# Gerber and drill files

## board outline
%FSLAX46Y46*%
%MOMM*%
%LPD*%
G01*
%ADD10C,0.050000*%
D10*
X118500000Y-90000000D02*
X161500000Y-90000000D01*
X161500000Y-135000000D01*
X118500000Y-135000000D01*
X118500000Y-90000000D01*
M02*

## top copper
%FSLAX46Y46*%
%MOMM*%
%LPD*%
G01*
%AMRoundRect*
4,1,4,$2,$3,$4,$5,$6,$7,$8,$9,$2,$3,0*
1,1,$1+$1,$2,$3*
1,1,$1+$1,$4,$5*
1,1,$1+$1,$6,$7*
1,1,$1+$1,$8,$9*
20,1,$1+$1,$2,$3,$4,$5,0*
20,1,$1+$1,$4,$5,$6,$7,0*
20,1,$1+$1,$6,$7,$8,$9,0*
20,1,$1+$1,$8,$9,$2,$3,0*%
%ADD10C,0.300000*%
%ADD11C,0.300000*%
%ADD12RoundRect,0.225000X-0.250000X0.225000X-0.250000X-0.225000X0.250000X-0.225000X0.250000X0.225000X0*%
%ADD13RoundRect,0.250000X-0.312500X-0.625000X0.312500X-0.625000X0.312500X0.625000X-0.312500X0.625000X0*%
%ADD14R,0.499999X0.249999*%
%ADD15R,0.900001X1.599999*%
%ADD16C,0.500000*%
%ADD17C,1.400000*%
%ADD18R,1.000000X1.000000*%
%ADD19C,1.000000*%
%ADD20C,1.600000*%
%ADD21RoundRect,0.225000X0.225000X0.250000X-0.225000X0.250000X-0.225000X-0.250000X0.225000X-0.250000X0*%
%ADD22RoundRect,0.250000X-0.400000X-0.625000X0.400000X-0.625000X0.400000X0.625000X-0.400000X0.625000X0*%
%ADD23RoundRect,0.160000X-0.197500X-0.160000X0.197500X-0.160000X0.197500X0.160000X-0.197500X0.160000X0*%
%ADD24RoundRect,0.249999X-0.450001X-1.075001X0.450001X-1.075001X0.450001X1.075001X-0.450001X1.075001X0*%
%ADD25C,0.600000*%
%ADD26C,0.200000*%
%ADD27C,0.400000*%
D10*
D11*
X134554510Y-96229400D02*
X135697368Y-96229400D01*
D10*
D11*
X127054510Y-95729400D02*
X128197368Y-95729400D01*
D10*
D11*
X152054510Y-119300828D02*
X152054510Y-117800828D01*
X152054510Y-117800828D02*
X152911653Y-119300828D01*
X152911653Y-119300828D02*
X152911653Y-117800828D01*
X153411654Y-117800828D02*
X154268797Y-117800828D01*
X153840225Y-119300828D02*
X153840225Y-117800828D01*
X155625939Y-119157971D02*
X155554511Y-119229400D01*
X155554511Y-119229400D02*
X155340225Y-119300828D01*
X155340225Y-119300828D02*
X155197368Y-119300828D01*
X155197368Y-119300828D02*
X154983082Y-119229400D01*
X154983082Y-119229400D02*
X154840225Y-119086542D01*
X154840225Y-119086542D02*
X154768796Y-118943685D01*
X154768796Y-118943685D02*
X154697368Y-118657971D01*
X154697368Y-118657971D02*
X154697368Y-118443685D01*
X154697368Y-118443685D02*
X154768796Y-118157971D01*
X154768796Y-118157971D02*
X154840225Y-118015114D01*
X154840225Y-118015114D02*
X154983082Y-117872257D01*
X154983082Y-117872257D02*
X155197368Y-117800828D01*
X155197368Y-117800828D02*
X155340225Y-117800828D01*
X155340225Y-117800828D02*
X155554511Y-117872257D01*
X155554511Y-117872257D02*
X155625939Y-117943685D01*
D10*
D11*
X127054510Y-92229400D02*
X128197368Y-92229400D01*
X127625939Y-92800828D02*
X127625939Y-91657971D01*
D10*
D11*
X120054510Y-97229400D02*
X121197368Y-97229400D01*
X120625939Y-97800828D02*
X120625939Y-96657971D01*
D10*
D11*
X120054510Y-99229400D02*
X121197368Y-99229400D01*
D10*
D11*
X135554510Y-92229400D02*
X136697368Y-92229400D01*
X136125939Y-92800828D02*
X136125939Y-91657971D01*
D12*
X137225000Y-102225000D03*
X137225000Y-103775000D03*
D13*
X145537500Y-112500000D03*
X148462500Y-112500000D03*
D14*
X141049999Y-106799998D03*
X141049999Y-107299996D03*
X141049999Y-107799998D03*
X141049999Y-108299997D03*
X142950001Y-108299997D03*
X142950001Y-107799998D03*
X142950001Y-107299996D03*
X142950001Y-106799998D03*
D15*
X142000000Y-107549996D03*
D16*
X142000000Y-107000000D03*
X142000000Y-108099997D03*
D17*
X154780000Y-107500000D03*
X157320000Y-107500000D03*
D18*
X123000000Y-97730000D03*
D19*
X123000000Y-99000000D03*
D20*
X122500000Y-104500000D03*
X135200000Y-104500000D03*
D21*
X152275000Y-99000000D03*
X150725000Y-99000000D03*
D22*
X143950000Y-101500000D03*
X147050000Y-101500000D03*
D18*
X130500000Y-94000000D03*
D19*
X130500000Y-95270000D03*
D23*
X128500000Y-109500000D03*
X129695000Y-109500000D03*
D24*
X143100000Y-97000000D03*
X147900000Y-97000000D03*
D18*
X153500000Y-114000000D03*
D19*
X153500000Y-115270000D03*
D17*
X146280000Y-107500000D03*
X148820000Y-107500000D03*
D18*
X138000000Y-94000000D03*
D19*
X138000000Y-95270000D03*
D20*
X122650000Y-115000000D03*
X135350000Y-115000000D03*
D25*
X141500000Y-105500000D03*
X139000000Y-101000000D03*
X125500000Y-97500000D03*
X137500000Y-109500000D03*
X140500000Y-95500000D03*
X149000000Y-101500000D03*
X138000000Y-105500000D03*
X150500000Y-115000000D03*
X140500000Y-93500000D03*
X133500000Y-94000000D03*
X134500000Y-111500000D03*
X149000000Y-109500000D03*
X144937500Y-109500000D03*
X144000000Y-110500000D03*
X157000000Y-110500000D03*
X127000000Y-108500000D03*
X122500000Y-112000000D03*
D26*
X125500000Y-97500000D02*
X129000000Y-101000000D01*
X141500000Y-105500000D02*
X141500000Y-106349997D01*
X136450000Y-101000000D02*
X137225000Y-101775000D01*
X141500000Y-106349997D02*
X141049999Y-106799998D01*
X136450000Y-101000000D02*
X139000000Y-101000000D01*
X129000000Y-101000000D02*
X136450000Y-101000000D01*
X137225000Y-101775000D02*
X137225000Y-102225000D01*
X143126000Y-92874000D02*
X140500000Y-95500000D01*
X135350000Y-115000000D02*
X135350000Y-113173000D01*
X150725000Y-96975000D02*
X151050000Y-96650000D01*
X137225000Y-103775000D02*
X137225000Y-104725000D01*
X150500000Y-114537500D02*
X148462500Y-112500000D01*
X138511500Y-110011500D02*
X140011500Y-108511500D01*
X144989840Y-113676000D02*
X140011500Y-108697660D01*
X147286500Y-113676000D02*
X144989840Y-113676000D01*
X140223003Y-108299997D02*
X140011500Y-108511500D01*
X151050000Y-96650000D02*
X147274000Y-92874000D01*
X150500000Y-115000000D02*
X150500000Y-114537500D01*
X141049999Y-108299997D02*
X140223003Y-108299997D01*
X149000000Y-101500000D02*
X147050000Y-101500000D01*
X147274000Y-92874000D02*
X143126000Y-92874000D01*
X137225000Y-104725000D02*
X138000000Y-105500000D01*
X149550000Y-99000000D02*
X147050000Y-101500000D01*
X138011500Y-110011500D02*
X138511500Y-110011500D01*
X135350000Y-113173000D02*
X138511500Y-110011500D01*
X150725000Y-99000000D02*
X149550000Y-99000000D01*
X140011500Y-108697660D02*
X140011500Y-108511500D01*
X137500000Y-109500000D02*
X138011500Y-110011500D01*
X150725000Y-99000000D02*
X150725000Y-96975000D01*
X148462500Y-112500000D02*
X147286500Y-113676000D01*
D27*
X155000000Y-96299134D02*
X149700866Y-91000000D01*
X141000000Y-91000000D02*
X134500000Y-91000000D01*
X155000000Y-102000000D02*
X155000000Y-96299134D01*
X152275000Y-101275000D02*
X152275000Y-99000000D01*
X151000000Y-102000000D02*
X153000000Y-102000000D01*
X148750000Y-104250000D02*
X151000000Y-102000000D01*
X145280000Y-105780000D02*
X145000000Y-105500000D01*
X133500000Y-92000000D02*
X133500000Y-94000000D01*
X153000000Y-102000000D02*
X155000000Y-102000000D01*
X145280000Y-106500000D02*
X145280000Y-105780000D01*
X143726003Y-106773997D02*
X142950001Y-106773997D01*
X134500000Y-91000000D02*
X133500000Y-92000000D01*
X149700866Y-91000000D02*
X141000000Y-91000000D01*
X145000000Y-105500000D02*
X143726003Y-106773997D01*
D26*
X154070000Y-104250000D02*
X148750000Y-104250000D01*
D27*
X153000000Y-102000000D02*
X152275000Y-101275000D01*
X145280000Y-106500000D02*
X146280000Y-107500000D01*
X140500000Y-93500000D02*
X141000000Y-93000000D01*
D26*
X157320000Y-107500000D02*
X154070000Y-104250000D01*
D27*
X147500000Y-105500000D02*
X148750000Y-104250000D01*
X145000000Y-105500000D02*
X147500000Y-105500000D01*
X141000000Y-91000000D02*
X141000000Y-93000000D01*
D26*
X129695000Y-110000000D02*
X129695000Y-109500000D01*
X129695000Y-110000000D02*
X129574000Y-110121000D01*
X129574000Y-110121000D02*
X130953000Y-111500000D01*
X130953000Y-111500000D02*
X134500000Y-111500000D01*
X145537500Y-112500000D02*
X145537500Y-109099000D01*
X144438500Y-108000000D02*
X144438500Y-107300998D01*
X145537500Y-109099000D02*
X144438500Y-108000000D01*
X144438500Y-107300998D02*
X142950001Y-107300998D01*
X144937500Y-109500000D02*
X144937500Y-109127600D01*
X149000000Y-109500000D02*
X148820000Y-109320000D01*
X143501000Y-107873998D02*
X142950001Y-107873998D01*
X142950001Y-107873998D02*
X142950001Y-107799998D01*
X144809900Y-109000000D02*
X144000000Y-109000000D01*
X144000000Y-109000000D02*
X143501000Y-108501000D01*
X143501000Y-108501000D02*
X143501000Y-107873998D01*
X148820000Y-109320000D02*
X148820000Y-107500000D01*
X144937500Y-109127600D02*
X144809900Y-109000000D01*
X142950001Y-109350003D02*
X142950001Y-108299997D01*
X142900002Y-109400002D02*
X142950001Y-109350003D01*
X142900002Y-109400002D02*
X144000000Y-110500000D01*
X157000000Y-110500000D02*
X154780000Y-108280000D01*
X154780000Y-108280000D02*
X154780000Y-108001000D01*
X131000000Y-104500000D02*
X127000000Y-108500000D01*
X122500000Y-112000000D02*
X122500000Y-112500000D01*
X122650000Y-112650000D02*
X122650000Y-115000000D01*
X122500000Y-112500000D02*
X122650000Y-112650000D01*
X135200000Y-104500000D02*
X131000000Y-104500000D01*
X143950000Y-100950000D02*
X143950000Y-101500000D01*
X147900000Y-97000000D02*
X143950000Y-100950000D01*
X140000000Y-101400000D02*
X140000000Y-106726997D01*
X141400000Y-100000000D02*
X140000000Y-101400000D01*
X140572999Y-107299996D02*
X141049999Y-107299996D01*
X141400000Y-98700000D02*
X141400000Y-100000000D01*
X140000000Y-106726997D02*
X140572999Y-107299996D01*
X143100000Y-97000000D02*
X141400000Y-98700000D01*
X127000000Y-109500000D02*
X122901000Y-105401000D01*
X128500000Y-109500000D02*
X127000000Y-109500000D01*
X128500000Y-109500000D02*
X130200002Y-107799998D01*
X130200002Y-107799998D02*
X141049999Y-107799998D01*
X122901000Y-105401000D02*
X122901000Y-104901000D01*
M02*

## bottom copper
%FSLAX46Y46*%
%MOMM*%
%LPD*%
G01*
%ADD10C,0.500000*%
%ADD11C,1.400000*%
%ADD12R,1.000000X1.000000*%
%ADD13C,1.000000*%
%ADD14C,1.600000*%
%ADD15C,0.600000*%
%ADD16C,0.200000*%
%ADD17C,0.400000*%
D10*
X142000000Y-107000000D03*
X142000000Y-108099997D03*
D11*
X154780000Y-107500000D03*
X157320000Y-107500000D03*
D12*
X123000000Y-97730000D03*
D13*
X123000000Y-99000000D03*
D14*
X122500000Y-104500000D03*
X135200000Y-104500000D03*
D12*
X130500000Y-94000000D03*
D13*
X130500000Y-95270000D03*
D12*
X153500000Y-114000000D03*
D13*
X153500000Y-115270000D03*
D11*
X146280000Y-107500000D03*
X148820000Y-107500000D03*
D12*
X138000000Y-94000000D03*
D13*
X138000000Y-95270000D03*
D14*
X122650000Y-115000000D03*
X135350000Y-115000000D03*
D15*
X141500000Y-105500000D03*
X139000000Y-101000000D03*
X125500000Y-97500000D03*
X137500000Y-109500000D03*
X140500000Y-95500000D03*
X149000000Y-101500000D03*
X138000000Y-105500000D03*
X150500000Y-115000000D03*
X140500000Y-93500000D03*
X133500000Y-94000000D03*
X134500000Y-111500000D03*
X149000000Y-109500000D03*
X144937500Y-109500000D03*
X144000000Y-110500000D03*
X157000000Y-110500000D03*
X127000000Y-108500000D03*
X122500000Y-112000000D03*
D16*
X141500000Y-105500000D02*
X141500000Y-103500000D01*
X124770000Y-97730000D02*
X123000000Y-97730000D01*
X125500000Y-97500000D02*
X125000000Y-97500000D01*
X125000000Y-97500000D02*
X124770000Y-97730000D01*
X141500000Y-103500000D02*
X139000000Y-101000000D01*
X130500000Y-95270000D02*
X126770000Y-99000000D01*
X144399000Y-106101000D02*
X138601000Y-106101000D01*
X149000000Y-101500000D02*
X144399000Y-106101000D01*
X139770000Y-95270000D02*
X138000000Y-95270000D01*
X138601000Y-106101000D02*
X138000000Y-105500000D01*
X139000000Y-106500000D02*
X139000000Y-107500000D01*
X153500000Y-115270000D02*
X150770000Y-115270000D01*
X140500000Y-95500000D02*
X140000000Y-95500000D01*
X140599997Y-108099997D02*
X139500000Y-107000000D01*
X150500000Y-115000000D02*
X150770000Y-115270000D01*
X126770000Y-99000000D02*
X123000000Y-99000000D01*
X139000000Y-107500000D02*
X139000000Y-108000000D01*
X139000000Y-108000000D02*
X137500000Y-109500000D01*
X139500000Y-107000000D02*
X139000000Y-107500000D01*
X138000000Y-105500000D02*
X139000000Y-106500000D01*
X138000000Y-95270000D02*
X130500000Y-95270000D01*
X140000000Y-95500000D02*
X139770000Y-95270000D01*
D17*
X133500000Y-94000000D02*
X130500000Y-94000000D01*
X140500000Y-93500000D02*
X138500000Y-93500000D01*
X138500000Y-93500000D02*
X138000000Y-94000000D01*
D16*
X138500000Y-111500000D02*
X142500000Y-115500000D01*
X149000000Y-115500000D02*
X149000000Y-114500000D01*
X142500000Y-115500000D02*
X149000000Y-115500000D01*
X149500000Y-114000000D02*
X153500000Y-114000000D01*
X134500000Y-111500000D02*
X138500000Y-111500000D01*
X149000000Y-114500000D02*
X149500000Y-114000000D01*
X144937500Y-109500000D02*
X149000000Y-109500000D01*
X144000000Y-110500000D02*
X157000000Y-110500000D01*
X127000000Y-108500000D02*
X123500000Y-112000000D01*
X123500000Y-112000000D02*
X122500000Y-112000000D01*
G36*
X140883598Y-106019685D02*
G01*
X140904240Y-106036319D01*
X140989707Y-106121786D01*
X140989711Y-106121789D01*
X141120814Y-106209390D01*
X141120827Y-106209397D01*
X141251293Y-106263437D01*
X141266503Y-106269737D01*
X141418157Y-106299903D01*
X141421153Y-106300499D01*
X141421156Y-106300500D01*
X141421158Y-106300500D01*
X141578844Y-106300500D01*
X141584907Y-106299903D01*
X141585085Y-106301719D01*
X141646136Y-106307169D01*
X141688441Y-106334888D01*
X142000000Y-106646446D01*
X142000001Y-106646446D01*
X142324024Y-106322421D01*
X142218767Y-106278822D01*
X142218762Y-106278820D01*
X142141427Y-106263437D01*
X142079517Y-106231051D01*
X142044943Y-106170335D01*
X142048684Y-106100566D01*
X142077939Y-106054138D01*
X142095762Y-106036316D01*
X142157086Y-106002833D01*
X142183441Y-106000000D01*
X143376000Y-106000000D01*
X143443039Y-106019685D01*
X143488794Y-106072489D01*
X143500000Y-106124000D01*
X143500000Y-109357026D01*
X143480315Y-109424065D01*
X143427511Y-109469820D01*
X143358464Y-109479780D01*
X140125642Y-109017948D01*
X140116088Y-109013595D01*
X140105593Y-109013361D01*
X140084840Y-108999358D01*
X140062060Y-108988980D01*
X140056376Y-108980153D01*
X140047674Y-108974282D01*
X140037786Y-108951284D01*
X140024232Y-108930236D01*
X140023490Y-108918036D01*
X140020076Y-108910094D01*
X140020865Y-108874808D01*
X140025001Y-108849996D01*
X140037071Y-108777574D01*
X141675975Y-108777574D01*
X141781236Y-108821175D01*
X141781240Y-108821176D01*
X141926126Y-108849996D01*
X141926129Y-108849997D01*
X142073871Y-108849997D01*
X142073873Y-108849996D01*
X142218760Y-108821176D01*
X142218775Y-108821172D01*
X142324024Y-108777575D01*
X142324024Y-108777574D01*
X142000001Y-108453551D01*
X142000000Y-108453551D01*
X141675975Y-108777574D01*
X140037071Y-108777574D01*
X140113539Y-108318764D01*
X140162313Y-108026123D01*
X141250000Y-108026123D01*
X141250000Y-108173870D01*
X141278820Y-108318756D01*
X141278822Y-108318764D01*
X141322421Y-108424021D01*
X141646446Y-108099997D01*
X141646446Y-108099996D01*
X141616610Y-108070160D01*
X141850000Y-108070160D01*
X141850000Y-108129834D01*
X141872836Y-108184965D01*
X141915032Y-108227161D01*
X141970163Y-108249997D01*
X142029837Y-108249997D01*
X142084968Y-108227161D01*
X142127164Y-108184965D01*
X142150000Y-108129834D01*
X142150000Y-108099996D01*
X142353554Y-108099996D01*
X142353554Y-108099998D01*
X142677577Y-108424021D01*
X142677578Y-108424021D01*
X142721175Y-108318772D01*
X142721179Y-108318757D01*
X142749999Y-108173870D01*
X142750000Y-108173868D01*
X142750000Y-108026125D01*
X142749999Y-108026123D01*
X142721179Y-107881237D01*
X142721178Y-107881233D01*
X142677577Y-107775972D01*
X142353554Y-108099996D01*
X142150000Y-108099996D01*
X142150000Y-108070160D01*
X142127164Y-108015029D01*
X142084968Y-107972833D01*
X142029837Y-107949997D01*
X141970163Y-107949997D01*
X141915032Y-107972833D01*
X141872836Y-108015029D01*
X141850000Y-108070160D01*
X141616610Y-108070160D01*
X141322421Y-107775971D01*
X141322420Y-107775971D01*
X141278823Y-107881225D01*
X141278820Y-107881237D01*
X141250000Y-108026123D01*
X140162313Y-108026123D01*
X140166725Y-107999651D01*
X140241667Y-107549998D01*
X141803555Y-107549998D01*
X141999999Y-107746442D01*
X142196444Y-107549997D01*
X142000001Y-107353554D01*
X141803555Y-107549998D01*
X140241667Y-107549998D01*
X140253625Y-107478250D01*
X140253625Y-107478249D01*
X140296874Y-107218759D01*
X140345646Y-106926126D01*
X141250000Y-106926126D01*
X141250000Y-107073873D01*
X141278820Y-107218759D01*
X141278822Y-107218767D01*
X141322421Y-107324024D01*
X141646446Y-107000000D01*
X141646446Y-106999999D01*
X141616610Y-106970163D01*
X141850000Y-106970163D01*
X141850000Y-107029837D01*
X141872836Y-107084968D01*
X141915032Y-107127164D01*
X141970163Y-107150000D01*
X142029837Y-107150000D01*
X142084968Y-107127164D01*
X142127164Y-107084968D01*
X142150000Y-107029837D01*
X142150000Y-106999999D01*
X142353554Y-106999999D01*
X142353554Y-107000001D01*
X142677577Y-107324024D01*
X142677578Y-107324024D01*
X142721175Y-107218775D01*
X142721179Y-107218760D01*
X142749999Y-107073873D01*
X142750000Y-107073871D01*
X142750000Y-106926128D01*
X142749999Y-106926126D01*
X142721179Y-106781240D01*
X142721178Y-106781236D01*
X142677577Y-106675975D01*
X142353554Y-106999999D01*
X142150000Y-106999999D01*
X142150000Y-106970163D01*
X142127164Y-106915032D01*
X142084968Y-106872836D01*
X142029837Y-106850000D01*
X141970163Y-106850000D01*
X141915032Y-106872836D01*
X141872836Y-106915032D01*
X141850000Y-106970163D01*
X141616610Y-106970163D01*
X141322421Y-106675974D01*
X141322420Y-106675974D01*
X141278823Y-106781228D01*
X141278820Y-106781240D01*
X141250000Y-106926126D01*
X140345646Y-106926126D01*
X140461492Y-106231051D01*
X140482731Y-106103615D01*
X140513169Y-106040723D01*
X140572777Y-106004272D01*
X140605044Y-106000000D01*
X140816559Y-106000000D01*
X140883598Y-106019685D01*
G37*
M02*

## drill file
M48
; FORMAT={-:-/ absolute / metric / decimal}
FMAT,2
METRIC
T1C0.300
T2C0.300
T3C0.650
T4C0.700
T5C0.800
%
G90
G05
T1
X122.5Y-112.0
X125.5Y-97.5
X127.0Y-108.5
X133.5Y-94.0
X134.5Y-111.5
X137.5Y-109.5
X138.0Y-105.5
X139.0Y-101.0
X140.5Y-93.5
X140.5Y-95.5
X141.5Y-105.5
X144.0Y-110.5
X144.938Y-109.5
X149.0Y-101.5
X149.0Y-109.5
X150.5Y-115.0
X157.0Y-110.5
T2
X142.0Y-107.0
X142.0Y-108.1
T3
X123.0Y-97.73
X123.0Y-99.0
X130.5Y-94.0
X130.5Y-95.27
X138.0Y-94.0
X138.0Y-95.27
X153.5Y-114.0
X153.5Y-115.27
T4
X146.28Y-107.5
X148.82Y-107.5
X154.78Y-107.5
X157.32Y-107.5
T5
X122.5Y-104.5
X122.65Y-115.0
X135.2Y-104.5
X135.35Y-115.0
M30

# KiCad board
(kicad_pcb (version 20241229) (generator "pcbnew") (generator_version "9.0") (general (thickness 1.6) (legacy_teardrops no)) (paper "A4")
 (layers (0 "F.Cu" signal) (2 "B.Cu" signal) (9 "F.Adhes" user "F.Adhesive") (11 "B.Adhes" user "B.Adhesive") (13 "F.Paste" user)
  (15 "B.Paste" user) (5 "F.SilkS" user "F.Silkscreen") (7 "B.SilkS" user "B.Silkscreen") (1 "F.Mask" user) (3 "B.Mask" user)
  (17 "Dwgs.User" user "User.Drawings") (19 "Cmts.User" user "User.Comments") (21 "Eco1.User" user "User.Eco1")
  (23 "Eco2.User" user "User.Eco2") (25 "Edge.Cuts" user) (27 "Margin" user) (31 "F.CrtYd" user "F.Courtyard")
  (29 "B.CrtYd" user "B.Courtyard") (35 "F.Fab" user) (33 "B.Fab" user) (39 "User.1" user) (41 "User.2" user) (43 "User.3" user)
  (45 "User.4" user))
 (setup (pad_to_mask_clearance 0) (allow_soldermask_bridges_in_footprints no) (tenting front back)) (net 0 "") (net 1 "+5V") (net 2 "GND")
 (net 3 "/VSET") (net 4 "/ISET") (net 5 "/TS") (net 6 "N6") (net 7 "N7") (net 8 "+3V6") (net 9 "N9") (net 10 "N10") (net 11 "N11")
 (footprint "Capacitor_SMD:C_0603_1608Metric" (layer "F.Cu") (at 137.225 103 -90)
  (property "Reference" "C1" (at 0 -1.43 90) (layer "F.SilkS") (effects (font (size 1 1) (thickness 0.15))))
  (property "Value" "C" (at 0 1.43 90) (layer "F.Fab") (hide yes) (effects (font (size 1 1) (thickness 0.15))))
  (pad "1" smd roundrect (at -0.775 0 270) (size 0.9 0.95) (layers "F.Cu" "F.Mask" "F.Paste") (roundrect_rratio 0.25) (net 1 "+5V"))
  (pad "2" smd roundrect (at 0.775 0 270) (size 0.9 0.95) (layers "F.Cu" "F.Mask" "F.Paste") (roundrect_rratio 0.25) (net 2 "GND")))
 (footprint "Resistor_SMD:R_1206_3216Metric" (layer "F.Cu") (at 147 112.5)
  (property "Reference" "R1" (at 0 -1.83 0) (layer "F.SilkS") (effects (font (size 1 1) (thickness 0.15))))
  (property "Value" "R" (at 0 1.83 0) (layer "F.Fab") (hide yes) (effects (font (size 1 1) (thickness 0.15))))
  (pad "1" smd roundrect (at -1.4625 0) (size 1.125 1.75) (layers "F.Cu" "F.Mask" "F.Paste") (roundrect_rratio 0.222222) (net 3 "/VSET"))
  (pad "2" smd roundrect (at 1.4625 0) (size 1.125 1.75) (layers "F.Cu" "F.Mask" "F.Paste") (roundrect_rratio 0.222222) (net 2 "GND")))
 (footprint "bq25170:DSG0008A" (layer "F.Cu") (at 142 107.549996)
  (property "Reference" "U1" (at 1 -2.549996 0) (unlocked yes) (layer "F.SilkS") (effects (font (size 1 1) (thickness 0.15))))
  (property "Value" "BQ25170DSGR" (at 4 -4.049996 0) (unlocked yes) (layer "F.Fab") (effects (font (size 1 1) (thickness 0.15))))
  (pad "1" smd rect (at -0.950001 -0.749998 90) (size 0.249999 0.499999) (layers "F.Cu" "F.Mask" "F.Paste") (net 1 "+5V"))
  (pad "2" smd rect (at -0.950001 -0.25 90) (size 0.249999 0.499999) (layers "F.Cu" "F.Mask" "F.Paste") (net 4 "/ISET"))
  (pad "3" smd rect (at -0.950001 0.250002 90) (size 0.249999 0.499999) (layers "F.Cu" "F.Mask" "F.Paste") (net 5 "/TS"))
  (pad "4" smd rect (at -0.950001 0.750001 90) (size 0.249999 0.499999) (layers "F.Cu" "F.Mask" "F.Paste") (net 2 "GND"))
  (pad "5" smd rect (at 0.950001 0.750001 90) (size 0.249999 0.499999) (layers "F.Cu" "F.Mask" "F.Paste") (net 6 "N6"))
  (pad "6" smd rect (at 0.950001 0.250002 90) (size 0.249999 0.499999) (layers "F.Cu" "F.Mask" "F.Paste") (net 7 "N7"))
  (pad "7" smd rect (at 0.950001 -0.25 90) (size 0.249999 0.499999) (layers "F.Cu" "F.Mask" "F.Paste") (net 3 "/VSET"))
  (pad "8" smd rect (at 0.950001 -0.749998 90) (size 0.249999 0.499999) (layers "F.Cu" "F.Mask" "F.Paste") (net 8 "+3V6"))
  (pad "9" smd rect (at 0 0) (size 0.900001 1.599999) (layers "F.Cu" "F.Mask" "F.Paste") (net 2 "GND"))
  (pad "10" thru_hole circle (at 0 -0.549996) (size 0.5 0.5) (drill 0.3) (layers "*.Cu" "*.Mask") (remove_unused_layers no) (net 2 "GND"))
  (pad "11" thru_hole circle (at 0 0.550001) (size 0.5 0.5) (drill 0.3) (layers "*.Cu" "*.Mask") (remove_unused_layers no) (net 2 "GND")))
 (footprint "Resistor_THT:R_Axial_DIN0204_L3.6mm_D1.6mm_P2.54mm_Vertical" (layer "F.Cu") (at 154.78 107.5)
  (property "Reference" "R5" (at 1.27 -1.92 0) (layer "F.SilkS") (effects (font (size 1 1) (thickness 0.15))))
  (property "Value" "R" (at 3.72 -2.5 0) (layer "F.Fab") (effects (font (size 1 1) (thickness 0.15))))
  (pad "1" thru_hole circle (at 0 0) (size 1.4 1.4) (drill 0.7) (layers "*.Cu" "*.Mask") (remove_unused_layers yes) (keep_end_layers yes)
   (zone_layer_connections) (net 6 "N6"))
  (pad "2" thru_hole circle (at 2.54 0) (size 1.4 1.4) (drill 0.7) (layers "*.Cu" "*.Mask") (remove_unused_layers yes) (keep_end_layers yes)
   (zone_layer_connections) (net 8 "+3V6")))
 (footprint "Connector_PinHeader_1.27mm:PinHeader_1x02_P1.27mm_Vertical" (layer "F.Cu") (at 123 97.73)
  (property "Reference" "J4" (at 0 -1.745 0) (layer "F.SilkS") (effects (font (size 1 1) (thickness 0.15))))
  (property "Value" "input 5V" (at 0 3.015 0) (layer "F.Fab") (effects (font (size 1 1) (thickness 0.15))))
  (pad "1" thru_hole rect (at 0 0) (size 1 1) (drill 0.65) (layers "*.Cu" "*.Mask") (remove_unused_layers no) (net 1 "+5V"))
  (pad "2" thru_hole circle (at 0 1.27) (size 1 1) (drill 0.65) (layers "*.Cu" "*.Mask") (remove_unused_layers no) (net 2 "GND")))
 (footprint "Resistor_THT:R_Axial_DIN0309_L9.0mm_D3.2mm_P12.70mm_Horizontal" (layer "F.Cu") (at 122.5 104.5)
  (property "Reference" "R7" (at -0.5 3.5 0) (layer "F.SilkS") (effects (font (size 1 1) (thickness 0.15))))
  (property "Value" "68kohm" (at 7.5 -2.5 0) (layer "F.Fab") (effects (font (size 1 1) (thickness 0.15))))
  (pad "1" thru_hole circle (at 0 0) (size 1.6 1.6) (drill 0.8) (layers "*.Cu" "*.Mask") (remove_unused_layers yes) (keep_end_layers yes)
   (zone_layer_connections) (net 5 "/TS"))
  (pad "2" thru_hole circle (at 12.7 0) (size 1.6 1.6) (drill 0.8) (layers "*.Cu" "*.Mask") (remove_unused_layers yes) (keep_end_layers yes)
   (zone_layer_connections) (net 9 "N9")))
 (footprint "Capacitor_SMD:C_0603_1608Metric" (layer "F.Cu") (at 151.5 99 180)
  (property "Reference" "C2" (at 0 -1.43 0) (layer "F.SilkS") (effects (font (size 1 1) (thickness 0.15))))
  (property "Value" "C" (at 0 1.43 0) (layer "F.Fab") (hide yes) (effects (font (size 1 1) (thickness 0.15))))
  (pad "1" smd roundrect (at -0.775 0 180) (size 0.9 0.95) (layers "F.Cu" "F.Mask" "F.Paste") (roundrect_rratio 0.25) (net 8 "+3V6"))
  (pad "2" smd roundrect (at 0.775 0 180) (size 0.9 0.95) (layers "F.Cu" "F.Mask" "F.Paste") (roundrect_rratio 0.25) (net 2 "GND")))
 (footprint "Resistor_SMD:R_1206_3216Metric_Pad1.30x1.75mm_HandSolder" (layer "F.Cu") (at 145.5 101.5)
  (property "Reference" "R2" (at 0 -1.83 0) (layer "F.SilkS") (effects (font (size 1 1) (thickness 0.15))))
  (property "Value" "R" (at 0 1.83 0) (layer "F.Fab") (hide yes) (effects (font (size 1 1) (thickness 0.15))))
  (pad "1" smd roundrect (at -1.55 0) (size 1.3 1.75) (layers "F.Cu" "F.Mask" "F.Paste") (roundrect_rratio 0.192308) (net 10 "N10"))
  (pad "2" smd roundrect (at 1.55 0) (size 1.3 1.75) (layers "F.Cu" "F.Mask" "F.Paste") (roundrect_rratio 0.192308) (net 2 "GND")))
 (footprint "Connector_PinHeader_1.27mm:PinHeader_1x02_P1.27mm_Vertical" (layer "F.Cu") (at 130.5 94)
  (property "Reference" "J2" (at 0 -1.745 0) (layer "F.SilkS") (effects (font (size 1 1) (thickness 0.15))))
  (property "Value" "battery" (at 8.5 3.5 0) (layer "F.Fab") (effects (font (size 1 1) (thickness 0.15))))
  (pad "1" thru_hole rect (at 0 0) (size 1 1) (drill 0.65) (layers "*.Cu" "*.Mask") (remove_unused_layers yes) (keep_end_layers yes)
   (zone_layer_connections) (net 8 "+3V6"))
  (pad "2" thru_hole circle (at 0 1.27) (size 1 1) (drill 0.65) (layers "*.Cu" "*.Mask") (remove_unused_layers yes) (keep_end_layers yes)
   (zone_layer_connections) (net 2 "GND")))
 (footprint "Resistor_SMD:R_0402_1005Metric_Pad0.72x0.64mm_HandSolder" (layer "F.Cu") (at 129.0975 109.5)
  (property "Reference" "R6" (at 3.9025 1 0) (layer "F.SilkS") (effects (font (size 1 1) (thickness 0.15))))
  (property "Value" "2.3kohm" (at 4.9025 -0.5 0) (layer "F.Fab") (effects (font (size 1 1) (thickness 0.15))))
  (pad "1" smd roundrect (at -0.5975 0) (size 0.715 0.64) (layers "F.Cu" "F.Mask" "F.Paste") (roundrect_rratio 0.25) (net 5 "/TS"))
  (pad "2" smd roundrect (at 0.5975 0) (size 0.715 0.64) (layers "F.Cu" "F.Mask" "F.Paste") (roundrect_rratio 0.25) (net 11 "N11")))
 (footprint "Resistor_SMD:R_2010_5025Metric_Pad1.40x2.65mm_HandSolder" (layer "F.Cu") (at 145.5 97)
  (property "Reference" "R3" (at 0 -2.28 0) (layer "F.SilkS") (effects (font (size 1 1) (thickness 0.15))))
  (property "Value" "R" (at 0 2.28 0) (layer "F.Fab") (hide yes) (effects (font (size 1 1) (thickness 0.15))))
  (pad "1" smd roundrect (at -2.4 0) (size 1.4 2.65) (layers "F.Cu" "F.Mask" "F.Paste") (roundrect_rratio 0.178571) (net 4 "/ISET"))
  (pad "2" smd roundrect (at 2.4 0) (size 1.4 2.65) (layers "F.Cu" "F.Mask" "F.Paste") (roundrect_rratio 0.178571) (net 10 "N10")))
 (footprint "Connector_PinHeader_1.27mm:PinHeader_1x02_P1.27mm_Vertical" (layer "F.Cu") (at 153.5 114)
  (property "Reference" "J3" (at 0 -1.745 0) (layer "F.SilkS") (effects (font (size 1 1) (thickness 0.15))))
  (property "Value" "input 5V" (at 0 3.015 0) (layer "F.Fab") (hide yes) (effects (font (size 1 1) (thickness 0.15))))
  (pad "1" thru_hole rect (at 0 0) (size 1 1) (drill 0.65) (layers "*.Cu" "*.Mask") (remove_unused_layers no) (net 11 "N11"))
  (pad "2" thru_hole circle (at 0 1.27) (size 1 1) (drill 0.65) (layers "*.Cu" "*.Mask") (remove_unused_layers no) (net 2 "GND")))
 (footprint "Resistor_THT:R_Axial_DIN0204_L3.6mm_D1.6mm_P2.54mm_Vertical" (layer "F.Cu") (at 146.28 107.5)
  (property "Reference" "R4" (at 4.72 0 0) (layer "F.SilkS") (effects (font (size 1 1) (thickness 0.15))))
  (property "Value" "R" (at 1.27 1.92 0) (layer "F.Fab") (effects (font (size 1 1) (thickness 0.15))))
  (pad "1" thru_hole circle (at 0 0) (size 1.4 1.4) (drill 0.7) (layers "*.Cu" "*.Mask") (remove_unused_layers yes) (keep_end_layers yes)
   (zone_layer_connections) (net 8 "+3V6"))
  (pad "2" thru_hole circle (at 2.54 0) (size 1.4 1.4) (drill 0.7) (layers "*.Cu" "*.Mask") (remove_unused_layers yes) (keep_end_layers yes)
   (zone_layer_connections) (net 7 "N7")))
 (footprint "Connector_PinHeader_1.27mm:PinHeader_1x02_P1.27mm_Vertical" (layer "F.Cu") (at 138 94)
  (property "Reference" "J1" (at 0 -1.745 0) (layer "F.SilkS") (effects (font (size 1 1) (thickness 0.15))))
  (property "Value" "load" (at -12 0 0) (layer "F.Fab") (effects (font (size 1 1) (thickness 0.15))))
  (pad "1" thru_hole rect (at 0 0) (size 1 1) (drill 0.65) (layers "*.Cu" "*.Mask") (remove_unused_layers yes) (keep_end_layers yes)
   (zone_layer_connections) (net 8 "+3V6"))
  (pad "2" thru_hole circle (at 0 1.27) (size 1 1) (drill 0.65) (layers "*.Cu" "*.Mask") (remove_unused_layers yes) (keep_end_layers yes)
   (zone_layer_connections) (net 2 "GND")))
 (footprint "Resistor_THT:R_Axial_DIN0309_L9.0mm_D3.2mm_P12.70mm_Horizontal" (layer "F.Cu") (at 122.65 115)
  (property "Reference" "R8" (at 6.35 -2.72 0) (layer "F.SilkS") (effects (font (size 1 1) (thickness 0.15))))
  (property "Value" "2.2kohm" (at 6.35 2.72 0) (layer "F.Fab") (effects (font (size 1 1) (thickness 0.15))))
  (pad "1" thru_hole circle (at 0 0) (size 1.6 1.6) (drill 0.8) (layers "*.Cu" "*.Mask") (remove_unused_layers yes) (keep_end_layers yes)
   (zone_layer_connections) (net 9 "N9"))
  (pad "2" thru_hole circle (at 12.7 0) (size 1.6 1.6) (drill 0.8) (layers "*.Cu" "*.Mask") (remove_unused_layers yes) (keep_end_layers yes)
   (zone_layer_connections) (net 2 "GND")))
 (gr_rect (start 118.5 90) (end 161.5 135) (stroke (width 0.05) (type default)) (fill no) (layer "Edge.Cuts"))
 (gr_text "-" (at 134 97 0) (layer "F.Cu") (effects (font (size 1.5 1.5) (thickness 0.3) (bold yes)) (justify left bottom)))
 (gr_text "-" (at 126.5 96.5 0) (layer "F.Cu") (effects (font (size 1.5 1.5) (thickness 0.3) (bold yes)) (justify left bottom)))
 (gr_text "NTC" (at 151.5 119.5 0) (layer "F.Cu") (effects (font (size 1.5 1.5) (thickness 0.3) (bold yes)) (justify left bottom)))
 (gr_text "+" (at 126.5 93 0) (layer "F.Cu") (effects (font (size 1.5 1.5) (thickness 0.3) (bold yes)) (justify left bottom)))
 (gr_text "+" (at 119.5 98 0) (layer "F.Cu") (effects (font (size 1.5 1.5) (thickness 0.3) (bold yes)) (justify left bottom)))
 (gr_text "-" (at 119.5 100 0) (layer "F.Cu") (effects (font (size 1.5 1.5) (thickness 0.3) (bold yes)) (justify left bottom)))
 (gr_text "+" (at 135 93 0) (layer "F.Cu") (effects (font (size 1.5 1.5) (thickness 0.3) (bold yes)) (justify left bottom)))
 (segment (start 125.5 97.5) (end 129 101) (width 0.2) (layer "F.Cu") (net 1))
 (segment (start 141.5 105.5) (end 141.5 106.349997) (width 0.2) (layer "F.Cu") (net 1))
 (segment (start 136.45 101) (end 137.225 101.775) (width 0.2) (layer "F.Cu") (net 1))
 (segment (start 141.5 106.349997) (end 141.049999 106.799998) (width 0.2) (layer "F.Cu") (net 1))
 (segment (start 136.45 101) (end 139 101) (width 0.2) (layer "F.Cu") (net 1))
 (segment (start 129 101) (end 136.45 101) (width 0.2) (layer "F.Cu") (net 1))
 (segment (start 137.225 101.775) (end 137.225 102.225) (width 0.2) (layer "F.Cu") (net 1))
 (via (at 141.5 105.5) (size 0.6) (drill 0.3) (layers "F.Cu" "B.Cu") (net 1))
 (via (at 139 101) (size 0.6) (drill 0.3) (layers "F.Cu" "B.Cu") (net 1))
 (via (at 125.5 97.5) (size 0.6) (drill 0.3) (layers "F.Cu" "B.Cu") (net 1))
 (segment (start 141.5 105.5) (end 141.5 103.5) (width 0.2) (layer "B.Cu") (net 1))
 (segment (start 124.77 97.73) (end 123 97.73) (width 0.2) (layer "B.Cu") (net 1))
 (segment (start 125.5 97.5) (end 125 97.5) (width 0.2) (layer "B.Cu") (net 1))
 (segment (start 125 97.5) (end 124.77 97.73) (width 0.2) (layer "B.Cu") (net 1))
 (segment (start 141.5 103.5) (end 139 101) (width 0.2) (layer "B.Cu") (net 1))
 (segment (start 143.126 92.874) (end 140.5 95.5) (width 0.2) (layer "F.Cu") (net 2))
 (segment (start 135.35 115) (end 135.35 113.173) (width 0.2) (layer "F.Cu") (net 2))
 (segment (start 150.725 96.975) (end 151.05 96.65) (width 0.2) (layer "F.Cu") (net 2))
 (segment (start 137.225 103.775) (end 137.225 104.725) (width 0.2) (layer "F.Cu") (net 2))
 (segment (start 150.5 114.5375) (end 148.4625 112.5) (width 0.2) (layer "F.Cu") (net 2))
 (segment (start 138.5115 110.0115) (end 140.0115 108.5115) (width 0.2) (layer "F.Cu") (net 2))
 (segment (start 144.98984 113.676) (end 140.0115 108.69766) (width 0.2) (layer "F.Cu") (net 2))
 (segment (start 147.2865 113.676) (end 144.98984 113.676) (width 0.2) (layer "F.Cu") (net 2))
 (segment (start 140.223003 108.299997) (end 140.0115 108.5115) (width 0.2) (layer "F.Cu") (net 2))
 (segment (start 151.05 96.65) (end 147.274 92.874) (width 0.2) (layer "F.Cu") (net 2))
 (segment (start 150.5 115) (end 150.5 114.5375) (width 0.2) (layer "F.Cu") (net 2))
 (segment (start 141.049999 108.299997) (end 140.223003 108.299997) (width 0.2) (layer "F.Cu") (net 2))
 (segment (start 149 101.5) (end 147.05 101.5) (width 0.2) (layer "F.Cu") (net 2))
 (segment (start 147.274 92.874) (end 143.126 92.874) (width 0.2) (layer "F.Cu") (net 2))
 (segment (start 137.225 104.725) (end 138 105.5) (width 0.2) (layer "F.Cu") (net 2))
 (segment (start 149.55 99) (end 147.05 101.5) (width 0.2) (layer "F.Cu") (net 2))
 (segment (start 138.0115 110.0115) (end 138.5115 110.0115) (width 0.2) (layer "F.Cu") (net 2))
 (segment (start 135.35 113.173) (end 138.5115 110.0115) (width 0.2) (layer "F.Cu") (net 2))
 (segment (start 150.725 99) (end 149.55 99) (width 0.2) (layer "F.Cu") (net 2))
 (segment (start 140.0115 108.69766) (end 140.0115 108.5115) (width 0.2) (layer "F.Cu") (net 2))
 (segment (start 137.5 109.5) (end 138.0115 110.0115) (width 0.2) (layer "F.Cu") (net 2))
 (segment (start 150.725 99) (end 150.725 96.975) (width 0.2) (layer "F.Cu") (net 2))
 (segment (start 148.4625 112.5) (end 147.2865 113.676) (width 0.2) (layer "F.Cu") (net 2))
 (via (at 137.5 109.5) (size 0.6) (drill 0.3) (layers "F.Cu" "B.Cu") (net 2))
 (via (at 140.5 95.5) (size 0.6) (drill 0.3) (layers "F.Cu" "B.Cu") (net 2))
 (via (at 149 101.5) (size 0.6) (drill 0.3) (layers "F.Cu" "B.Cu") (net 2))
 (via (at 138 105.5) (size 0.6) (drill 0.3) (layers "F.Cu" "B.Cu") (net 2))
 (via (at 150.5 115) (size 0.6) (drill 0.3) (layers "F.Cu" "B.Cu") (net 2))
 (segment (start 130.5 95.27) (end 126.77 99) (width 0.2) (layer "B.Cu") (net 2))
 (segment (start 144.399 106.101) (end 138.601 106.101) (width 0.2) (layer "B.Cu") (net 2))
 (segment (start 149 101.5) (end 144.399 106.101) (width 0.2) (layer "B.Cu") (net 2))
 (segment (start 139.77 95.27) (end 138 95.27) (width 0.2) (layer "B.Cu") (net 2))
 (segment (start 138.601 106.101) (end 138 105.5) (width 0.2) (layer "B.Cu") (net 2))
 (segment (start 139 106.5) (end 139 107.5) (width 0.2) (layer "B.Cu") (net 2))
 (segment (start 153.5 115.27) (end 150.77 115.27) (width 0.2) (layer "B.Cu") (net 2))
 (segment (start 140.5 95.5) (end 140 95.5) (width 0.2) (layer "B.Cu") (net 2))
 (segment (start 140.599997 108.099997) (end 139.5 107) (width 0.2) (layer "B.Cu") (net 2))
 (segment (start 150.5 115) (end 150.77 115.27) (width 0.2) (layer "B.Cu") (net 2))
 (segment (start 126.77 99) (end 123 99) (width 0.2) (layer "B.Cu") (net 2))
 (segment (start 139 107.5) (end 139 108) (width 0.2) (layer "B.Cu") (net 2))
 (segment (start 139 108) (end 137.5 109.5) (width 0.2) (layer "B.Cu") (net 2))
 (segment (start 139.5 107) (end 139 107.5) (width 0.2) (layer "B.Cu") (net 2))
 (segment (start 138 105.5) (end 139 106.5) (width 0.2) (layer "B.Cu") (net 2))
 (segment (start 138 95.27) (end 130.5 95.27) (width 0.2) (layer "B.Cu") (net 2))
 (segment (start 140 95.5) (end 139.77 95.27) (width 0.2) (layer "B.Cu") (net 2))
 (segment (start 155 96.299134) (end 149.700866 91) (width 0.4) (layer "F.Cu") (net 8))
 (segment (start 141 91) (end 134.5 91) (width 0.4) (layer "F.Cu") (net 8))
 (segment (start 155 102) (end 155 96.299134) (width 0.4) (layer "F.Cu") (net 8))
 (segment (start 152.275 101.275) (end 152.275 99) (width 0.4) (layer "F.Cu") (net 8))
 (segment (start 151 102) (end 153 102) (width 0.4) (layer "F.Cu") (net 8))
 (segment (start 148.75 104.25) (end 151 102) (width 0.4) (layer "F.Cu") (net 8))
 (segment (start 145.28 105.78) (end 145 105.5) (width 0.4) (layer "F.Cu") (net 8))
 (segment (start 133.5 92) (end 133.5 94) (width 0.4) (layer "F.Cu") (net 8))
 (segment (start 153 102) (end 155 102) (width 0.4) (layer "F.Cu") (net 8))
 (segment (start 145.28 106.5) (end 145.28 105.78) (width 0.4) (layer "F.Cu") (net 8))
 (segment (start 143.726003 106.773997) (end 142.950001 106.773997) (width 0.4) (layer "F.Cu") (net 8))
 (segment (start 134.5 91) (end 133.5 92) (width 0.4) (layer "F.Cu") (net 8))
 (segment (start 149.700866 91) (end 141 91) (width 0.4) (layer "F.Cu") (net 8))
 (segment (start 145 105.5) (end 143.726003 106.773997) (width 0.4) (layer "F.Cu") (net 8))
 (segment (start 154.07 104.25) (end 148.75 104.25) (width 0.2) (layer "F.Cu") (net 8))
 (segment (start 153 102) (end 152.275 101.275) (width 0.4) (layer "F.Cu") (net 8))
 (segment (start 145.28 106.5) (end 146.28 107.5) (width 0.4) (layer "F.Cu") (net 8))
 (segment (start 140.5 93.5) (end 141 93) (width 0.4) (layer "F.Cu") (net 8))
 (segment (start 157.32 107.5) (end 154.07 104.25) (width 0.2) (layer "F.Cu") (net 8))
 (segment (start 147.5 105.5) (end 148.75 104.25) (width 0.4) (layer "F.Cu") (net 8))
 (segment (start 145 105.5) (end 147.5 105.5) (width 0.4) (layer "F.Cu") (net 8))
 (segment (start 141 91) (end 141 93) (width 0.4) (layer "F.Cu") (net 8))
 (via (at 140.5 93.5) (size 0.6) (drill 0.3) (layers "F.Cu" "B.Cu") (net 8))
 (via (at 133.5 94) (size 0.6) (drill 0.3) (layers "F.Cu" "B.Cu") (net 8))
 (segment (start 133.5 94) (end 130.5 94) (width 0.4) (layer "B.Cu") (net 8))
 (segment (start 140.5 93.5) (end 138.5 93.5) (width 0.4) (layer "B.Cu") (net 8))
 (segment (start 138.5 93.5) (end 138 94) (width 0.4) (layer "B.Cu") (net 8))
 (segment (start 129.695 110) (end 129.695 109.5) (width 0.2) (layer "F.Cu") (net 11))
 (segment (start 129.695 110) (end 129.574 110.121) (width 0.2) (layer "F.Cu") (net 11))
 (segment (start 129.574 110.121) (end 130.953 111.5) (width 0.2) (layer "F.Cu") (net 11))
 (segment (start 130.953 111.5) (end 134.5 111.5) (width 0.2) (layer "F.Cu") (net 11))
 (via (at 134.5 111.5) (size 0.6) (drill 0.3) (layers "F.Cu" "B.Cu") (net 11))
 (segment (start 138.5 111.5) (end 142.5 115.5) (width 0.2) (layer "B.Cu") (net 11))
 (segment (start 149 115.5) (end 149 114.5) (width 0.2) (layer "B.Cu") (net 11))
 (segment (start 142.5 115.5) (end 149 115.5) (width 0.2) (layer "B.Cu") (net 11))
 (segment (start 149.5 114) (end 153.5 114) (width 0.2) (layer "B.Cu") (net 11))
 (segment (start 134.5 111.5) (end 138.5 111.5) (width 0.2) (layer "B.Cu") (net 11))
 (segment (start 149 114.5) (end 149.5 114) (width 0.2) (layer "B.Cu") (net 11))
 (segment (start 145.5375 112.5) (end 145.5375 109.099) (width 0.2) (layer "F.Cu") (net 3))
 (segment (start 144.4385 108) (end 144.4385 107.300998) (width 0.2) (layer "F.Cu") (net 3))
 (segment (start 145.5375 109.099) (end 144.4385 108) (width 0.2) (layer "F.Cu") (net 3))
 (segment (start 144.4385 107.300998) (end 142.950001 107.300998) (width 0.2) (layer "F.Cu") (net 3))
 (segment (start 144.9375 109.5) (end 144.9375 109.1276) (width 0.2) (layer "F.Cu") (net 7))
 (segment (start 149 109.5) (end 148.82 109.32) (width 0.2) (layer "F.Cu") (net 7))
 (segment (start 143.501 107.873998) (end 142.950001 107.873998) (width 0.2) (layer "F.Cu") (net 7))
 (segment (start 142.950001 107.873998) (end 142.950001 107.799998) (width 0.2) (layer "F.Cu") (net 7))
 (segment (start 144.8099 109) (end 144 109) (width 0.2) (layer "F.Cu") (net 7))
 (segment (start 144 109) (end 143.501 108.501) (width 0.2) (layer "F.Cu") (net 7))
 (segment (start 143.501 108.501) (end 143.501 107.873998) (width 0.2) (layer "F.Cu") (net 7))
 (segment (start 148.82 109.32) (end 148.82 107.5) (width 0.2) (layer "F.Cu") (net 7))
 (segment (start 144.9375 109.1276) (end 144.8099 109) (width 0.2) (layer "F.Cu") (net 7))
 (via (at 149 109.5) (size 0.6) (drill 0.3) (layers "F.Cu" "B.Cu") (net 7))
 (via (at 144.9375 109.5) (size 0.6) (drill 0.3) (layers "F.Cu" "B.Cu") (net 7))
 (segment (start 144.9375 109.5) (end 149 109.5) (width 0.2) (layer "B.Cu") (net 7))
 (segment (start 142.950001 109.350003) (end 142.950001 108.299997) (width 0.2) (layer "F.Cu") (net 6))
 (segment (start 142.900002 109.400002) (end 142.950001 109.350003) (width 0.2) (layer "F.Cu") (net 6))
 (segment (start 142.900002 109.400002) (end 144 110.5) (width 0.2) (layer "F.Cu") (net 6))
 (segment (start 157 110.5) (end 154.78 108.28) (width 0.2) (layer "F.Cu") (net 6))
 (segment (start 154.78 108.28) (end 154.78 108.001) (width 0.2) (layer "F.Cu") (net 6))
 (via (at 144 110.5) (size 0.6) (drill 0.3) (layers "F.Cu" "B.Cu") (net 6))
 (via (at 157 110.5) (size 0.6) (drill 0.3) (layers "F.Cu" "B.Cu") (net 6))
 (segment (start 144 110.5) (end 157 110.5) (width 0.2) (layer "B.Cu") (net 6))
 (segment (start 131 104.5) (end 127 108.5) (width 0.2) (layer "F.Cu") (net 9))
 (segment (start 122.5 112) (end 122.5 112.5) (width 0.2) (layer "F.Cu") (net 9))
 (segment (start 122.65 112.65) (end 122.65 115) (width 0.2) (layer "F.Cu") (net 9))
 (segment (start 122.5 112.5) (end 122.65 112.65) (width 0.2) (layer "F.Cu") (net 9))
 (segment (start 135.2 104.5) (end 131 104.5) (width 0.2) (layer "F.Cu") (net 9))
 (via (at 127 108.5) (size 0.6) (drill 0.3) (layers "F.Cu" "B.Cu") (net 9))
 (via (at 122.5 112) (size 0.6) (drill 0.3) (layers "F.Cu" "B.Cu") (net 9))
 (segment (start 127 108.5) (end 123.5 112) (width 0.2) (layer "B.Cu") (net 9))
 (segment (start 123.5 112) (end 122.5 112) (width 0.2) (layer "B.Cu") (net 9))
 (segment (start 143.95 100.95) (end 143.95 101.5) (width 0.2) (layer "F.Cu") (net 10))
 (segment (start 147.9 97) (end 143.95 100.95) (width 0.2) (layer "F.Cu") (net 10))
 (segment (start 140 101.4) (end 140 106.726997) (width 0.2) (layer "F.Cu") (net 4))
 (segment (start 141.4 100) (end 140 101.4) (width 0.2) (layer "F.Cu") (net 4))
 (segment (start 140.572999 107.299996) (end 141.049999 107.299996) (width 0.2) (layer "F.Cu") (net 4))
 (segment (start 141.4 98.7) (end 141.4 100) (width 0.2) (layer "F.Cu") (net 4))
 (segment (start 140 106.726997) (end 140.572999 107.299996) (width 0.2) (layer "F.Cu") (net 4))
 (segment (start 143.1 97) (end 141.4 98.7) (width 0.2) (layer "F.Cu") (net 4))
 (segment (start 127 109.5) (end 122.901 105.401) (width 0.2) (layer "F.Cu") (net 5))
 (segment (start 128.5 109.5) (end 127 109.5) (width 0.2) (layer "F.Cu") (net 5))
 (segment (start 128.5 109.5) (end 130.200002 107.799998) (width 0.2) (layer "F.Cu") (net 5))
 (segment (start 130.200002 107.799998) (end 141.049999 107.799998) (width 0.2) (layer "F.Cu") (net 5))
 (segment (start 122.901 105.401) (end 122.901 104.901) (width 0.2) (layer "F.Cu") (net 5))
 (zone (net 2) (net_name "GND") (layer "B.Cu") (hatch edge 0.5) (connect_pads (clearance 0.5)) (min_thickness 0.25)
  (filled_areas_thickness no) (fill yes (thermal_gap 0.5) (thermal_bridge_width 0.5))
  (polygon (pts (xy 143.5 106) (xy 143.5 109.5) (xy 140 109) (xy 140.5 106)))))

